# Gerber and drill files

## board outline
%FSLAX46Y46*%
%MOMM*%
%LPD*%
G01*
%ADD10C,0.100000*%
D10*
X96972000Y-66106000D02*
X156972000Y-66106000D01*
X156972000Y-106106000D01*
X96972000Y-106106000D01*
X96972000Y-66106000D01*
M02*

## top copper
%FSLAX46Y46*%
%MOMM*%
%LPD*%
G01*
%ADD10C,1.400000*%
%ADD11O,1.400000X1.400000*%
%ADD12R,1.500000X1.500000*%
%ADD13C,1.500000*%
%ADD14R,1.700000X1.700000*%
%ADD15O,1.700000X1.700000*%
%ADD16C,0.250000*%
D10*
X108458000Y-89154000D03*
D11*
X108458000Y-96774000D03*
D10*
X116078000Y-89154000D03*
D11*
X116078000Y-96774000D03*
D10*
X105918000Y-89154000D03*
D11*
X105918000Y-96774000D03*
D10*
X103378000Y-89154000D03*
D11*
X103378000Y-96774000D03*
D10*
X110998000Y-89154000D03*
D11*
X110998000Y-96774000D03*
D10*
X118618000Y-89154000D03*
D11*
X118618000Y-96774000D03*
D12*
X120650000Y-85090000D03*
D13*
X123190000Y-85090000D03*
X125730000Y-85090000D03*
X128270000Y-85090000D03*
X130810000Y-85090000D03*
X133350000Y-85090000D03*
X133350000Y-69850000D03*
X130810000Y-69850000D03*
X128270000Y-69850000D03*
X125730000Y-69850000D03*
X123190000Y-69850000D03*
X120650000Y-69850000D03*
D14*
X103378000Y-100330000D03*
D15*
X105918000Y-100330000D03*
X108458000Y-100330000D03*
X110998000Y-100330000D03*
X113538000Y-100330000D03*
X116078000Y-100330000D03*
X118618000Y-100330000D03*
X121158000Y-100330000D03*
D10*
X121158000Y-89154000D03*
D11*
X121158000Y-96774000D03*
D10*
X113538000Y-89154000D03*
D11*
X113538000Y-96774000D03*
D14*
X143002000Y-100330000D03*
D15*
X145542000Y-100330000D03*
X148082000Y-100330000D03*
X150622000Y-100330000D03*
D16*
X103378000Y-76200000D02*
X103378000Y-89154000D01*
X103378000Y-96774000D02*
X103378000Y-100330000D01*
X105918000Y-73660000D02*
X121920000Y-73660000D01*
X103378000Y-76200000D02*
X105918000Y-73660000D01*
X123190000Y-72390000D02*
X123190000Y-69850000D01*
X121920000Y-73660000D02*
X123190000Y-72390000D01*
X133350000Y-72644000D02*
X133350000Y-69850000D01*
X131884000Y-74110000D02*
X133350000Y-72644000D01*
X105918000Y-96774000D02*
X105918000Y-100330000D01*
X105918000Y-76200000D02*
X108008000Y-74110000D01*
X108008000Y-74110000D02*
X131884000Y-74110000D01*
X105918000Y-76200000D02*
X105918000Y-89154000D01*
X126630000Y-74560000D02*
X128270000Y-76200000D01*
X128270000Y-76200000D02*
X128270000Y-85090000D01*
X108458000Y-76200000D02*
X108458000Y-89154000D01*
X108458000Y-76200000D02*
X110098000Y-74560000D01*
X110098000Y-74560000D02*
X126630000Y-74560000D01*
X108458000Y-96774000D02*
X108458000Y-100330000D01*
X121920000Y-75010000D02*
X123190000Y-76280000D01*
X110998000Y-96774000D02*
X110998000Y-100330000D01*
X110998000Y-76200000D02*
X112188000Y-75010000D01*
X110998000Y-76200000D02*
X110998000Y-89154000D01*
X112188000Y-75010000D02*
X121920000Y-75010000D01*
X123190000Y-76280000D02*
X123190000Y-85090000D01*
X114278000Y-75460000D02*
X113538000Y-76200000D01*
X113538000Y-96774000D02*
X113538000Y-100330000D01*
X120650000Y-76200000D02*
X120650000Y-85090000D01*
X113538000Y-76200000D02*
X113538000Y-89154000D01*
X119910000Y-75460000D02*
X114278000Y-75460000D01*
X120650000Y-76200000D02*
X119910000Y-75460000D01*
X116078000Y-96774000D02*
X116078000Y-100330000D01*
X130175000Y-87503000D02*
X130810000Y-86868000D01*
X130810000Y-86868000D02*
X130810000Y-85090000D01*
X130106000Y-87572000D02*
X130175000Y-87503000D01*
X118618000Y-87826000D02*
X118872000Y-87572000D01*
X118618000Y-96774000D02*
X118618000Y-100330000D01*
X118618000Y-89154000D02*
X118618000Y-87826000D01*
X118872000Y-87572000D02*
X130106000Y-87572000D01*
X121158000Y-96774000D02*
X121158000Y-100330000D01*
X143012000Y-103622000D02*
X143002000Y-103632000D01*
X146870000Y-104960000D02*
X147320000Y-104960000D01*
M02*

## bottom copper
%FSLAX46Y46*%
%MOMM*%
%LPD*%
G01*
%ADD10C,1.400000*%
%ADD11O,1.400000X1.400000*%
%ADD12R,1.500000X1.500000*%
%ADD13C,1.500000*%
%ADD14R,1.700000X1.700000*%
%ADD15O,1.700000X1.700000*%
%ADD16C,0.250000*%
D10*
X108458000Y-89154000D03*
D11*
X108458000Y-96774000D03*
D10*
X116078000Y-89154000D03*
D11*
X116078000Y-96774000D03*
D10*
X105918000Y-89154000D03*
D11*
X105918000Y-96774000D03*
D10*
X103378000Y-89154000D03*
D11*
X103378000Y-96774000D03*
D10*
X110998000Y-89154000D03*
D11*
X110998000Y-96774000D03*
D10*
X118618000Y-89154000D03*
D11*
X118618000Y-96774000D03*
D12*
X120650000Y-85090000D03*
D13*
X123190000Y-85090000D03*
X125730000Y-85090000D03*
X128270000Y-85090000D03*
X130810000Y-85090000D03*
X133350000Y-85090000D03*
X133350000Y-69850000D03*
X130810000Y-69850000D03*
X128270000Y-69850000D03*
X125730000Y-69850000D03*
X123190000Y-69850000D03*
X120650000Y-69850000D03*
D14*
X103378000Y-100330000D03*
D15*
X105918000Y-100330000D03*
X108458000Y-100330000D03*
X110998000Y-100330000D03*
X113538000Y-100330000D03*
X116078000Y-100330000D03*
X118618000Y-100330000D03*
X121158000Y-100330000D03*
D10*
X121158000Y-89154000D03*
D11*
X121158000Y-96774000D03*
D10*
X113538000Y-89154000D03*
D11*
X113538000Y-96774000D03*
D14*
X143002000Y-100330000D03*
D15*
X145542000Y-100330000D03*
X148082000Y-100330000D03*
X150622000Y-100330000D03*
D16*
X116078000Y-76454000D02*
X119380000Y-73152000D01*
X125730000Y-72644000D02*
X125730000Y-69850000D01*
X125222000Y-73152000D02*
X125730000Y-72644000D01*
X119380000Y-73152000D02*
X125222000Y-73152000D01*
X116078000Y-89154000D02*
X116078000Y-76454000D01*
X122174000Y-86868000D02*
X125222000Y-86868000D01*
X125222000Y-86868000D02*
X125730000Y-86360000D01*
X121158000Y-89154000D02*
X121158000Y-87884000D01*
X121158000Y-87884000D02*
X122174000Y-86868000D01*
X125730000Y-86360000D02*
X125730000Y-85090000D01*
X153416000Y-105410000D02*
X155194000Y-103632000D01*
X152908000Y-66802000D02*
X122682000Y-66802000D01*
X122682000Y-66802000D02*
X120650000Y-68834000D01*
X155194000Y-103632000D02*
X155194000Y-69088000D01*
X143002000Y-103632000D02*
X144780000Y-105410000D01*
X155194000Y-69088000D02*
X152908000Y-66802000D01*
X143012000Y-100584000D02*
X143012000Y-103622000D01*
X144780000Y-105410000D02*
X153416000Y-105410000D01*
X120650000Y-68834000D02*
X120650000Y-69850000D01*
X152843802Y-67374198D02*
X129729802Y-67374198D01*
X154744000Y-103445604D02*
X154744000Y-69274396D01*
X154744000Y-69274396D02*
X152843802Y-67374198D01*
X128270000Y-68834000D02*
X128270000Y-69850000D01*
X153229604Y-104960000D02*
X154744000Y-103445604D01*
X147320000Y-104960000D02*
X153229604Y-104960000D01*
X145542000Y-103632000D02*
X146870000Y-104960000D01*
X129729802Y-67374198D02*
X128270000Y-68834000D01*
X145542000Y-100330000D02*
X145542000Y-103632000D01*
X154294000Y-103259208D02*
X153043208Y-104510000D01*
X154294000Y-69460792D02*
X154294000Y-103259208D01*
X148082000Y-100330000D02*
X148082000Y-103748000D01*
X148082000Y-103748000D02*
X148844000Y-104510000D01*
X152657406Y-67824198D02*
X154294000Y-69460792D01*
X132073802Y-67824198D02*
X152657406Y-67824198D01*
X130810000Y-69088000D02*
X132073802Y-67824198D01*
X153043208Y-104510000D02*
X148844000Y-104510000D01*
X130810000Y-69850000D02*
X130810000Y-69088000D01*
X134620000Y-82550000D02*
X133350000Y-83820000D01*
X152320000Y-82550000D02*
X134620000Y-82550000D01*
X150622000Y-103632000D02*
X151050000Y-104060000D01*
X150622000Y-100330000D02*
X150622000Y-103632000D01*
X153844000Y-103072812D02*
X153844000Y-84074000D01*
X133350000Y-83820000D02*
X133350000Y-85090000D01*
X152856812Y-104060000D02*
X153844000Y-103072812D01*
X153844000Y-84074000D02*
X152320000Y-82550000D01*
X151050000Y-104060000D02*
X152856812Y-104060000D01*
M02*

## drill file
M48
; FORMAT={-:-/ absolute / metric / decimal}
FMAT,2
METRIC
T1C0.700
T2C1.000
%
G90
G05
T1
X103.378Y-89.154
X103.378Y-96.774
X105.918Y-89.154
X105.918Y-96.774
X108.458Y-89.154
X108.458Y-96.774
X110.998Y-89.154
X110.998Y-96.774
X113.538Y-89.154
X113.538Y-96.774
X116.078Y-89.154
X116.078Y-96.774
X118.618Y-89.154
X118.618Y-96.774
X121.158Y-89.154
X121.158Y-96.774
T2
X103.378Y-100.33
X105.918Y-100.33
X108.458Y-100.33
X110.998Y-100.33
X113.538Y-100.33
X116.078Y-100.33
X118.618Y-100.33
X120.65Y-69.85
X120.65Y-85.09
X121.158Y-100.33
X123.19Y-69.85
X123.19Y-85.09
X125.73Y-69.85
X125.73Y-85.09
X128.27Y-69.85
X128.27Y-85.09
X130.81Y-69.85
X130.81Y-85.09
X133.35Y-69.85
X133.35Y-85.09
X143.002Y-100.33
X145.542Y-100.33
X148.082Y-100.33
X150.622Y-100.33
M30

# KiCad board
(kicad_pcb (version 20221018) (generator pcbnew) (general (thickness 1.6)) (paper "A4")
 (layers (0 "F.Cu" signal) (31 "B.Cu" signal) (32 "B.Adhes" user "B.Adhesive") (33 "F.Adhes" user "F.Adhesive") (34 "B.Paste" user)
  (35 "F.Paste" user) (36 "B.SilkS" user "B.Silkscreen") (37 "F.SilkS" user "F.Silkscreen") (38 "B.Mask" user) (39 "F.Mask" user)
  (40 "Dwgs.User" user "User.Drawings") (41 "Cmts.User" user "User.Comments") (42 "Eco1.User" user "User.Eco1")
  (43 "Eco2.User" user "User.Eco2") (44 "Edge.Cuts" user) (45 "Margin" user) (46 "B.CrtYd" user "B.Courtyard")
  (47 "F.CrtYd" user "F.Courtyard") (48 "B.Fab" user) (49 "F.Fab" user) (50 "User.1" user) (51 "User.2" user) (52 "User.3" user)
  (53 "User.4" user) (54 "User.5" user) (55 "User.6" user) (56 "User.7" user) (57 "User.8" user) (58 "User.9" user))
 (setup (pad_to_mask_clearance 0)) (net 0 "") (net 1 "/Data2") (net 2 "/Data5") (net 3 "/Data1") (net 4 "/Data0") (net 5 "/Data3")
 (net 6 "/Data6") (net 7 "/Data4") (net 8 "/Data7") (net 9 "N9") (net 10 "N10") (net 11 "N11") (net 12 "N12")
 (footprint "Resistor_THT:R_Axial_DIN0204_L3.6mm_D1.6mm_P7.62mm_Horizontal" (layer "F.Cu") (at 108.458 89.154 -90)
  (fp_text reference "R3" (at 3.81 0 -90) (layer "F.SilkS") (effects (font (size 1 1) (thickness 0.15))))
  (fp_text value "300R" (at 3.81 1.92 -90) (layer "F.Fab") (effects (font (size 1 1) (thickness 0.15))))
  (pad "1" thru_hole circle (at 0 0 270) (size 1.4 1.4) (drill 0.7) (layers "*.Cu" "*.Mask") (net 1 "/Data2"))
  (pad "2" thru_hole oval (at 7.62 0 270) (size 1.4 1.4) (drill 0.7) (layers "*.Cu" "*.Mask") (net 1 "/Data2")))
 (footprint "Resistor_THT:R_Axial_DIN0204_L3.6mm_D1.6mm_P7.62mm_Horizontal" (layer "F.Cu") (at 116.078 89.154 -90)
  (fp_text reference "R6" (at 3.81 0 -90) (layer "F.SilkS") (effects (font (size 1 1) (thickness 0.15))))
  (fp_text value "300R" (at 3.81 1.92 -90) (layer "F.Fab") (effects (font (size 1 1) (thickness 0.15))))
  (pad "1" thru_hole circle (at 0 0 270) (size 1.4 1.4) (drill 0.7) (layers "*.Cu" "*.Mask") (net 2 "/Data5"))
  (pad "2" thru_hole oval (at 7.62 0 270) (size 1.4 1.4) (drill 0.7) (layers "*.Cu" "*.Mask") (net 2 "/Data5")))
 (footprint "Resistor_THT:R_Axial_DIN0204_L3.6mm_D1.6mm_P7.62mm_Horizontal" (layer "F.Cu") (at 105.918 89.154 -90)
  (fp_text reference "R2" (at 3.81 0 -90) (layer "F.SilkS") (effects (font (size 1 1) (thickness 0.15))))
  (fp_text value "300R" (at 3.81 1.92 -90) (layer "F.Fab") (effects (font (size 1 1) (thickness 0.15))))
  (pad "1" thru_hole circle (at 0 0 270) (size 1.4 1.4) (drill 0.7) (layers "*.Cu" "*.Mask") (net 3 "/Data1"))
  (pad "2" thru_hole oval (at 7.62 0 270) (size 1.4 1.4) (drill 0.7) (layers "*.Cu" "*.Mask") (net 3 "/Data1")))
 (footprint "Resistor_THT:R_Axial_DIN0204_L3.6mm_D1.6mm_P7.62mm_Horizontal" (layer "F.Cu") (at 103.378 89.154 -90)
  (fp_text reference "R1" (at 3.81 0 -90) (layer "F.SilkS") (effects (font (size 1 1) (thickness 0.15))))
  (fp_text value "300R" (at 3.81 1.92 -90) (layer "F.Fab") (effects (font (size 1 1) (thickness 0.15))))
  (pad "1" thru_hole circle (at 0 0 270) (size 1.4 1.4) (drill 0.7) (layers "*.Cu" "*.Mask") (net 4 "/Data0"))
  (pad "2" thru_hole oval (at 7.62 0 270) (size 1.4 1.4) (drill 0.7) (layers "*.Cu" "*.Mask") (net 4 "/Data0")))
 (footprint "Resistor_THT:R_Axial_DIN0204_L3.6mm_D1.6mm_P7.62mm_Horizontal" (layer "F.Cu") (at 110.998 89.154 -90)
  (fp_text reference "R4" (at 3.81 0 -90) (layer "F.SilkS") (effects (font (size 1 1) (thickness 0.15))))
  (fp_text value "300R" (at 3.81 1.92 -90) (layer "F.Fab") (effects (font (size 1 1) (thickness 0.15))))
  (pad "1" thru_hole circle (at 0 0 270) (size 1.4 1.4) (drill 0.7) (layers "*.Cu" "*.Mask") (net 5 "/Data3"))
  (pad "2" thru_hole oval (at 7.62 0 270) (size 1.4 1.4) (drill 0.7) (layers "*.Cu" "*.Mask") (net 5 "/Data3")))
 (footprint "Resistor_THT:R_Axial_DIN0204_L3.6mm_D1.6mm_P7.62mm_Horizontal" (layer "F.Cu") (at 118.618 89.154 -90)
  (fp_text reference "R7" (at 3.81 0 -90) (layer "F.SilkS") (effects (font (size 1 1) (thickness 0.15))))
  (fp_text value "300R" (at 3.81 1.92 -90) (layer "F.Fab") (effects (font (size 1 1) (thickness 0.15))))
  (pad "1" thru_hole circle (at 0 0 270) (size 1.4 1.4) (drill 0.7) (layers "*.Cu" "*.Mask") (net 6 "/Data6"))
  (pad "2" thru_hole oval (at 7.62 0 270) (size 1.4 1.4) (drill 0.7) (layers "*.Cu" "*.Mask") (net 6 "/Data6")))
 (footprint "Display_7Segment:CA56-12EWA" (layer "F.Cu") (at 120.65 85.09 90)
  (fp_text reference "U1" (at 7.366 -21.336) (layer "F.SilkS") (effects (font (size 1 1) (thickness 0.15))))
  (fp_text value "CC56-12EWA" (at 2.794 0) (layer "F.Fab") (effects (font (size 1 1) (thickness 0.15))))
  (pad "1" thru_hole rect (at 0 0 90) (size 1.5 1.5) (drill 1) (layers "*.Cu" "*.Mask") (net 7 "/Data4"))
  (pad "2" thru_hole circle (at 0 2.54 90) (size 1.5 1.5) (drill 1) (layers "*.Cu" "*.Mask") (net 5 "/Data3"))
  (pad "3" thru_hole circle (at 0 5.08 90) (size 1.5 1.5) (drill 1) (layers "*.Cu" "*.Mask") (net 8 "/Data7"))
  (pad "4" thru_hole circle (at 0 7.62 90) (size 1.5 1.5) (drill 1) (layers "*.Cu" "*.Mask") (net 1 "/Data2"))
  (pad "5" thru_hole circle (at 0 10.16 90) (size 1.5 1.5) (drill 1) (layers "*.Cu" "*.Mask") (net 6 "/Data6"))
  (pad "6" thru_hole circle (at 0 12.7 90) (size 1.5 1.5) (drill 1) (layers "*.Cu" "*.Mask") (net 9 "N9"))
  (pad "7" thru_hole circle (at 15.24 12.7 90) (size 1.5 1.5) (drill 1) (layers "*.Cu" "*.Mask") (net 3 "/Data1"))
  (pad "8" thru_hole circle (at 15.24 10.16 90) (size 1.5 1.5) (drill 1) (layers "*.Cu" "*.Mask") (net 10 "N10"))
  (pad "9" thru_hole circle (at 15.24 7.62 90) (size 1.5 1.5) (drill 1) (layers "*.Cu" "*.Mask") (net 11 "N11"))
  (pad "10" thru_hole circle (at 15.24 5.08 90) (size 1.5 1.5) (drill 1) (layers "*.Cu" "*.Mask") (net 2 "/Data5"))
  (pad "11" thru_hole circle (at 15.24 2.54 90) (size 1.5 1.5) (drill 1) (layers "*.Cu" "*.Mask") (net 4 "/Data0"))
  (pad "12" thru_hole circle (at 15.24 0 90) (size 1.5 1.5) (drill 1) (layers "*.Cu" "*.Mask") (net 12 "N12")))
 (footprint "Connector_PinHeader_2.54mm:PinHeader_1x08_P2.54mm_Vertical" (layer "F.Cu") (at 103.378 100.33 90)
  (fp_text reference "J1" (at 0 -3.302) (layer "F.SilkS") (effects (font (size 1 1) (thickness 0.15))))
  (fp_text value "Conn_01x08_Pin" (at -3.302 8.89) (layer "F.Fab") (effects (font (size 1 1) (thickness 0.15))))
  (pad "1" thru_hole rect (at 0 0 90) (size 1.7 1.7) (drill 1) (layers "*.Cu" "*.Mask") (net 4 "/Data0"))
  (pad "2" thru_hole oval (at 0 2.54 90) (size 1.7 1.7) (drill 1) (layers "*.Cu" "*.Mask") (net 3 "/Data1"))
  (pad "3" thru_hole oval (at 0 5.08 90) (size 1.7 1.7) (drill 1) (layers "*.Cu" "*.Mask") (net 1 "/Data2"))
  (pad "4" thru_hole oval (at 0 7.62 90) (size 1.7 1.7) (drill 1) (layers "*.Cu" "*.Mask") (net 5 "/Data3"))
  (pad "5" thru_hole oval (at 0 10.16 90) (size 1.7 1.7) (drill 1) (layers "*.Cu" "*.Mask") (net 7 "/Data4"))
  (pad "6" thru_hole oval (at 0 12.7 90) (size 1.7 1.7) (drill 1) (layers "*.Cu" "*.Mask") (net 2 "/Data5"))
  (pad "7" thru_hole oval (at 0 15.24 90) (size 1.7 1.7) (drill 1) (layers "*.Cu" "*.Mask") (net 6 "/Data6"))
  (pad "8" thru_hole oval (at 0 17.78 90) (size 1.7 1.7) (drill 1) (layers "*.Cu" "*.Mask") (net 8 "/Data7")))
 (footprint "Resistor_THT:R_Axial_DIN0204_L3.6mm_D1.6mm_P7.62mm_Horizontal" (layer "F.Cu") (at 121.158 89.154 -90)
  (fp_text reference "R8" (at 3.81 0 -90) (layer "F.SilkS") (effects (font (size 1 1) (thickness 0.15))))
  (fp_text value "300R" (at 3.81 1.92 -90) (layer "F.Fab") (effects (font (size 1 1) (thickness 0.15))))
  (pad "1" thru_hole circle (at 0 0 270) (size 1.4 1.4) (drill 0.7) (layers "*.Cu" "*.Mask") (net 8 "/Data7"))
  (pad "2" thru_hole oval (at 7.62 0 270) (size 1.4 1.4) (drill 0.7) (layers "*.Cu" "*.Mask") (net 8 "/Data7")))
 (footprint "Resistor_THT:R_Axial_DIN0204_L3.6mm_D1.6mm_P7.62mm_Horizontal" (layer "F.Cu") (at 113.538 89.154 -90)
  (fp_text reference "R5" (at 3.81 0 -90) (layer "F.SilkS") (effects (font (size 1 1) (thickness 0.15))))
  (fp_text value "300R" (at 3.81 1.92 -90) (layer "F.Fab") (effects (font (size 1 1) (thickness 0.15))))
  (pad "1" thru_hole circle (at 0 0 270) (size 1.4 1.4) (drill 0.7) (layers "*.Cu" "*.Mask") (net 7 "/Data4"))
  (pad "2" thru_hole oval (at 7.62 0 270) (size 1.4 1.4) (drill 0.7) (layers "*.Cu" "*.Mask") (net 7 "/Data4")))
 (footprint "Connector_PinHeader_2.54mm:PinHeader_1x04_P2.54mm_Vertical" (layer "F.Cu") (at 143.002 100.33 90)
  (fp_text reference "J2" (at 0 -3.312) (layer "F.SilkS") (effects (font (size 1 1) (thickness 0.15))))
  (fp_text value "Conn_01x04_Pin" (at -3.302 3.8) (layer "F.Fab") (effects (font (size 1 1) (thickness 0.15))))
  (pad "1" thru_hole rect (at 0 0 90) (size 1.7 1.7) (drill 1) (layers "*.Cu" "*.Mask") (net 12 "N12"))
  (pad "2" thru_hole oval (at 0 2.54 90) (size 1.7 1.7) (drill 1) (layers "*.Cu" "*.Mask") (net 11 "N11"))
  (pad "3" thru_hole oval (at 0 5.08 90) (size 1.7 1.7) (drill 1) (layers "*.Cu" "*.Mask") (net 10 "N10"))
  (pad "4" thru_hole oval (at 0 7.62 90) (size 1.7 1.7) (drill 1) (layers "*.Cu" "*.Mask") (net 9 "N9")))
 (gr_rect (start 96.972 66.106) (end 156.972 106.106) (stroke (width 0.1) (type default)) (fill none) (layer "Edge.Cuts"))
 (segment (start 103.378 76.2) (end 103.378 89.154) (width 0.25) (layer "F.Cu") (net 4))
 (segment (start 103.378 96.774) (end 103.378 100.33) (width 0.25) (layer "F.Cu") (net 4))
 (segment (start 105.918 73.66) (end 121.92 73.66) (width 0.25) (layer "F.Cu") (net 4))
 (segment (start 103.378 76.2) (end 105.918 73.66) (width 0.25) (layer "F.Cu") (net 4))
 (segment (start 123.19 72.39) (end 123.19 69.85) (width 0.25) (layer "F.Cu") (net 4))
 (segment (start 121.92 73.66) (end 123.19 72.39) (width 0.25) (layer "F.Cu") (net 4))
 (segment (start 133.35 72.644) (end 133.35 69.85) (width 0.25) (layer "F.Cu") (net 3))
 (segment (start 131.884 74.11) (end 133.35 72.644) (width 0.25) (layer "F.Cu") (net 3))
 (segment (start 105.918 96.774) (end 105.918 100.33) (width 0.25) (layer "F.Cu") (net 3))
 (segment (start 105.918 76.2) (end 108.008 74.11) (width 0.25) (layer "F.Cu") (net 3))
 (segment (start 108.008 74.11) (end 131.884 74.11) (width 0.25) (layer "F.Cu") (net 3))
 (segment (start 105.918 76.2) (end 105.918 89.154) (width 0.25) (layer "F.Cu") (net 3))
 (segment (start 126.63 74.56) (end 128.27 76.2) (width 0.25) (layer "F.Cu") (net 1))
 (segment (start 128.27 76.2) (end 128.27 85.09) (width 0.25) (layer "F.Cu") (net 1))
 (segment (start 108.458 76.2) (end 108.458 89.154) (width 0.25) (layer "F.Cu") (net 1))
 (segment (start 108.458 76.2) (end 110.098 74.56) (width 0.25) (layer "F.Cu") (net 1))
 (segment (start 110.098 74.56) (end 126.63 74.56) (width 0.25) (layer "F.Cu") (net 1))
 (segment (start 108.458 96.774) (end 108.458 100.33) (width 0.25) (layer "F.Cu") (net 1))
 (segment (start 121.92 75.01) (end 123.19 76.28) (width 0.25) (layer "F.Cu") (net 5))
 (segment (start 110.998 96.774) (end 110.998 100.33) (width 0.25) (layer "F.Cu") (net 5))
 (segment (start 110.998 76.2) (end 112.188 75.01) (width 0.25) (layer "F.Cu") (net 5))
 (segment (start 110.998 76.2) (end 110.998 89.154) (width 0.25) (layer "F.Cu") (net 5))
 (segment (start 112.188 75.01) (end 121.92 75.01) (width 0.25) (layer "F.Cu") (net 5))
 (segment (start 123.19 76.28) (end 123.19 85.09) (width 0.25) (layer "F.Cu") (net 5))
 (segment (start 114.278 75.46) (end 113.538 76.2) (width 0.25) (layer "F.Cu") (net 7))
 (segment (start 113.538 96.774) (end 113.538 100.33) (width 0.25) (layer "F.Cu") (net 7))
 (segment (start 120.65 76.2) (end 120.65 85.09) (width 0.25) (layer "F.Cu") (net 7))
 (segment (start 113.538 76.2) (end 113.538 89.154) (width 0.25) (layer "F.Cu") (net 7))
 (segment (start 119.91 75.46) (end 114.278 75.46) (width 0.25) (layer "F.Cu") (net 7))
 (segment (start 120.65 76.2) (end 119.91 75.46) (width 0.25) (layer "F.Cu") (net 7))
 (segment (start 116.078 96.774) (end 116.078 100.33) (width 0.25) (layer "F.Cu") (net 2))
 (segment (start 116.078 76.454) (end 119.38 73.152) (width 0.25) (layer "B.Cu") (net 2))
 (segment (start 125.73 72.644) (end 125.73 69.85) (width 0.25) (layer "B.Cu") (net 2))
 (segment (start 125.222 73.152) (end 125.73 72.644) (width 0.25) (layer "B.Cu") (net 2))
 (segment (start 119.38 73.152) (end 125.222 73.152) (width 0.25) (layer "B.Cu") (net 2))
 (segment (start 116.078 89.154) (end 116.078 76.454) (width 0.25) (layer "B.Cu") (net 2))
 (segment (start 130.175 87.503) (end 130.81 86.868) (width 0.25) (layer "F.Cu") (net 6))
 (segment (start 130.81 86.868) (end 130.81 85.09) (width 0.25) (layer "F.Cu") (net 6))
 (segment (start 130.106 87.572) (end 130.175 87.503) (width 0.25) (layer "F.Cu") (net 6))
 (segment (start 118.618 87.826) (end 118.872 87.572) (width 0.25) (layer "F.Cu") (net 6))
 (segment (start 118.618 96.774) (end 118.618 100.33) (width 0.25) (layer "F.Cu") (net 6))
 (segment (start 118.618 89.154) (end 118.618 87.826) (width 0.25) (layer "F.Cu") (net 6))
 (segment (start 118.872 87.572) (end 130.106 87.572) (width 0.25) (layer "F.Cu") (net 6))
 (segment (start 121.158 96.774) (end 121.158 100.33) (width 0.25) (layer "F.Cu") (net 8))
 (segment (start 122.174 86.868) (end 125.222 86.868) (width 0.25) (layer "B.Cu") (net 8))
 (segment (start 125.222 86.868) (end 125.73 86.36) (width 0.25) (layer "B.Cu") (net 8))
 (segment (start 121.158 89.154) (end 121.158 87.884) (width 0.25) (layer "B.Cu") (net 8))
 (segment (start 121.158 87.884) (end 122.174 86.868) (width 0.25) (layer "B.Cu") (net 8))
 (segment (start 125.73 86.36) (end 125.73 85.09) (width 0.25) (layer "B.Cu") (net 8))
 (segment (start 143.012 103.622) (end 143.002 103.632) (width 0.25) (layer "F.Cu") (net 12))
 (segment (start 153.416 105.41) (end 155.194 103.632) (width 0.25) (layer "B.Cu") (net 12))
 (segment (start 152.908 66.802) (end 122.682 66.802) (width 0.25) (layer "B.Cu") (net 12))
 (segment (start 122.682 66.802) (end 120.65 68.834) (width 0.25) (layer "B.Cu") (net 12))
 (segment (start 155.194 103.632) (end 155.194 69.088) (width 0.25) (layer "B.Cu") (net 12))
 (segment (start 143.002 103.632) (end 144.78 105.41) (width 0.25) (layer "B.Cu") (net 12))
 (segment (start 155.194 69.088) (end 152.908 66.802) (width 0.25) (layer "B.Cu") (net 12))
 (segment (start 143.012 100.584) (end 143.012 103.622) (width 0.25) (layer "B.Cu") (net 12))
 (segment (start 144.78 105.41) (end 153.416 105.41) (width 0.25) (layer "B.Cu") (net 12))
 (segment (start 120.65 68.834) (end 120.65 69.85) (width 0.25) (layer "B.Cu") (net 12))
 (segment (start 146.87 104.96) (end 147.32 104.96) (width 0.25) (layer "F.Cu") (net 11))
 (segment (start 152.843802 67.374198) (end 129.729802 67.374198) (width 0.25) (layer "B.Cu") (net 11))
 (segment (start 154.744 103.445604) (end 154.744 69.274396) (width 0.25) (layer "B.Cu") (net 11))
 (segment (start 154.744 69.274396) (end 152.843802 67.374198) (width 0.25) (layer "B.Cu") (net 11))
 (segment (start 128.27 68.834) (end 128.27 69.85) (width 0.25) (layer "B.Cu") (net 11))
 (segment (start 153.229604 104.96) (end 154.744 103.445604) (width 0.25) (layer "B.Cu") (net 11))
 (segment (start 147.32 104.96) (end 153.229604 104.96) (width 0.25) (layer "B.Cu") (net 11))
 (segment (start 145.542 103.632) (end 146.87 104.96) (width 0.25) (layer "B.Cu") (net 11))
 (segment (start 129.729802 67.374198) (end 128.27 68.834) (width 0.25) (layer "B.Cu") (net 11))
 (segment (start 145.542 100.33) (end 145.542 103.632) (width 0.25) (layer "B.Cu") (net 11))
 (segment (start 154.294 103.259208) (end 153.043208 104.51) (width 0.25) (layer "B.Cu") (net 10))
 (segment (start 154.294 69.460792) (end 154.294 103.259208) (width 0.25) (layer "B.Cu") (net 10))
 (segment (start 148.082 100.33) (end 148.082 103.748) (width 0.25) (layer "B.Cu") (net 10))
 (segment (start 148.082 103.748) (end 148.844 104.51) (width 0.25) (layer "B.Cu") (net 10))
 (segment (start 152.657406 67.824198) (end 154.294 69.460792) (width 0.25) (layer "B.Cu") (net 10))
 (segment (start 132.073802 67.824198) (end 152.657406 67.824198) (width 0.25) (layer "B.Cu") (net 10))
 (segment (start 130.81 69.088) (end 132.073802 67.824198) (width 0.25) (layer "B.Cu") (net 10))
 (segment (start 153.043208 104.51) (end 148.844 104.51) (width 0.25) (layer "B.Cu") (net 10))
 (segment (start 130.81 69.85) (end 130.81 69.088) (width 0.25) (layer "B.Cu") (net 10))
 (segment (start 134.62 82.55) (end 133.35 83.82) (width 0.25) (layer "B.Cu") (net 9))
 (segment (start 152.32 82.55) (end 134.62 82.55) (width 0.25) (layer "B.Cu") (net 9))
 (segment (start 150.622 103.632) (end 151.05 104.06) (width 0.25) (layer "B.Cu") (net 9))
 (segment (start 150.622 100.33) (end 150.622 103.632) (width 0.25) (layer "B.Cu") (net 9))
 (segment (start 153.844 103.072812) (end 153.844 84.074) (width 0.25) (layer "B.Cu") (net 9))
 (segment (start 133.35 83.82) (end 133.35 85.09) (width 0.25) (layer "B.Cu") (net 9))
 (segment (start 152.856812 104.06) (end 153.844 103.072812) (width 0.25) (layer "B.Cu") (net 9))
 (segment (start 153.844 84.074) (end 152.32 82.55) (width 0.25) (layer "B.Cu") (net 9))
 (segment (start 151.05 104.06) (end 152.856812 104.06) (width 0.25) (layer "B.Cu") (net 9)))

